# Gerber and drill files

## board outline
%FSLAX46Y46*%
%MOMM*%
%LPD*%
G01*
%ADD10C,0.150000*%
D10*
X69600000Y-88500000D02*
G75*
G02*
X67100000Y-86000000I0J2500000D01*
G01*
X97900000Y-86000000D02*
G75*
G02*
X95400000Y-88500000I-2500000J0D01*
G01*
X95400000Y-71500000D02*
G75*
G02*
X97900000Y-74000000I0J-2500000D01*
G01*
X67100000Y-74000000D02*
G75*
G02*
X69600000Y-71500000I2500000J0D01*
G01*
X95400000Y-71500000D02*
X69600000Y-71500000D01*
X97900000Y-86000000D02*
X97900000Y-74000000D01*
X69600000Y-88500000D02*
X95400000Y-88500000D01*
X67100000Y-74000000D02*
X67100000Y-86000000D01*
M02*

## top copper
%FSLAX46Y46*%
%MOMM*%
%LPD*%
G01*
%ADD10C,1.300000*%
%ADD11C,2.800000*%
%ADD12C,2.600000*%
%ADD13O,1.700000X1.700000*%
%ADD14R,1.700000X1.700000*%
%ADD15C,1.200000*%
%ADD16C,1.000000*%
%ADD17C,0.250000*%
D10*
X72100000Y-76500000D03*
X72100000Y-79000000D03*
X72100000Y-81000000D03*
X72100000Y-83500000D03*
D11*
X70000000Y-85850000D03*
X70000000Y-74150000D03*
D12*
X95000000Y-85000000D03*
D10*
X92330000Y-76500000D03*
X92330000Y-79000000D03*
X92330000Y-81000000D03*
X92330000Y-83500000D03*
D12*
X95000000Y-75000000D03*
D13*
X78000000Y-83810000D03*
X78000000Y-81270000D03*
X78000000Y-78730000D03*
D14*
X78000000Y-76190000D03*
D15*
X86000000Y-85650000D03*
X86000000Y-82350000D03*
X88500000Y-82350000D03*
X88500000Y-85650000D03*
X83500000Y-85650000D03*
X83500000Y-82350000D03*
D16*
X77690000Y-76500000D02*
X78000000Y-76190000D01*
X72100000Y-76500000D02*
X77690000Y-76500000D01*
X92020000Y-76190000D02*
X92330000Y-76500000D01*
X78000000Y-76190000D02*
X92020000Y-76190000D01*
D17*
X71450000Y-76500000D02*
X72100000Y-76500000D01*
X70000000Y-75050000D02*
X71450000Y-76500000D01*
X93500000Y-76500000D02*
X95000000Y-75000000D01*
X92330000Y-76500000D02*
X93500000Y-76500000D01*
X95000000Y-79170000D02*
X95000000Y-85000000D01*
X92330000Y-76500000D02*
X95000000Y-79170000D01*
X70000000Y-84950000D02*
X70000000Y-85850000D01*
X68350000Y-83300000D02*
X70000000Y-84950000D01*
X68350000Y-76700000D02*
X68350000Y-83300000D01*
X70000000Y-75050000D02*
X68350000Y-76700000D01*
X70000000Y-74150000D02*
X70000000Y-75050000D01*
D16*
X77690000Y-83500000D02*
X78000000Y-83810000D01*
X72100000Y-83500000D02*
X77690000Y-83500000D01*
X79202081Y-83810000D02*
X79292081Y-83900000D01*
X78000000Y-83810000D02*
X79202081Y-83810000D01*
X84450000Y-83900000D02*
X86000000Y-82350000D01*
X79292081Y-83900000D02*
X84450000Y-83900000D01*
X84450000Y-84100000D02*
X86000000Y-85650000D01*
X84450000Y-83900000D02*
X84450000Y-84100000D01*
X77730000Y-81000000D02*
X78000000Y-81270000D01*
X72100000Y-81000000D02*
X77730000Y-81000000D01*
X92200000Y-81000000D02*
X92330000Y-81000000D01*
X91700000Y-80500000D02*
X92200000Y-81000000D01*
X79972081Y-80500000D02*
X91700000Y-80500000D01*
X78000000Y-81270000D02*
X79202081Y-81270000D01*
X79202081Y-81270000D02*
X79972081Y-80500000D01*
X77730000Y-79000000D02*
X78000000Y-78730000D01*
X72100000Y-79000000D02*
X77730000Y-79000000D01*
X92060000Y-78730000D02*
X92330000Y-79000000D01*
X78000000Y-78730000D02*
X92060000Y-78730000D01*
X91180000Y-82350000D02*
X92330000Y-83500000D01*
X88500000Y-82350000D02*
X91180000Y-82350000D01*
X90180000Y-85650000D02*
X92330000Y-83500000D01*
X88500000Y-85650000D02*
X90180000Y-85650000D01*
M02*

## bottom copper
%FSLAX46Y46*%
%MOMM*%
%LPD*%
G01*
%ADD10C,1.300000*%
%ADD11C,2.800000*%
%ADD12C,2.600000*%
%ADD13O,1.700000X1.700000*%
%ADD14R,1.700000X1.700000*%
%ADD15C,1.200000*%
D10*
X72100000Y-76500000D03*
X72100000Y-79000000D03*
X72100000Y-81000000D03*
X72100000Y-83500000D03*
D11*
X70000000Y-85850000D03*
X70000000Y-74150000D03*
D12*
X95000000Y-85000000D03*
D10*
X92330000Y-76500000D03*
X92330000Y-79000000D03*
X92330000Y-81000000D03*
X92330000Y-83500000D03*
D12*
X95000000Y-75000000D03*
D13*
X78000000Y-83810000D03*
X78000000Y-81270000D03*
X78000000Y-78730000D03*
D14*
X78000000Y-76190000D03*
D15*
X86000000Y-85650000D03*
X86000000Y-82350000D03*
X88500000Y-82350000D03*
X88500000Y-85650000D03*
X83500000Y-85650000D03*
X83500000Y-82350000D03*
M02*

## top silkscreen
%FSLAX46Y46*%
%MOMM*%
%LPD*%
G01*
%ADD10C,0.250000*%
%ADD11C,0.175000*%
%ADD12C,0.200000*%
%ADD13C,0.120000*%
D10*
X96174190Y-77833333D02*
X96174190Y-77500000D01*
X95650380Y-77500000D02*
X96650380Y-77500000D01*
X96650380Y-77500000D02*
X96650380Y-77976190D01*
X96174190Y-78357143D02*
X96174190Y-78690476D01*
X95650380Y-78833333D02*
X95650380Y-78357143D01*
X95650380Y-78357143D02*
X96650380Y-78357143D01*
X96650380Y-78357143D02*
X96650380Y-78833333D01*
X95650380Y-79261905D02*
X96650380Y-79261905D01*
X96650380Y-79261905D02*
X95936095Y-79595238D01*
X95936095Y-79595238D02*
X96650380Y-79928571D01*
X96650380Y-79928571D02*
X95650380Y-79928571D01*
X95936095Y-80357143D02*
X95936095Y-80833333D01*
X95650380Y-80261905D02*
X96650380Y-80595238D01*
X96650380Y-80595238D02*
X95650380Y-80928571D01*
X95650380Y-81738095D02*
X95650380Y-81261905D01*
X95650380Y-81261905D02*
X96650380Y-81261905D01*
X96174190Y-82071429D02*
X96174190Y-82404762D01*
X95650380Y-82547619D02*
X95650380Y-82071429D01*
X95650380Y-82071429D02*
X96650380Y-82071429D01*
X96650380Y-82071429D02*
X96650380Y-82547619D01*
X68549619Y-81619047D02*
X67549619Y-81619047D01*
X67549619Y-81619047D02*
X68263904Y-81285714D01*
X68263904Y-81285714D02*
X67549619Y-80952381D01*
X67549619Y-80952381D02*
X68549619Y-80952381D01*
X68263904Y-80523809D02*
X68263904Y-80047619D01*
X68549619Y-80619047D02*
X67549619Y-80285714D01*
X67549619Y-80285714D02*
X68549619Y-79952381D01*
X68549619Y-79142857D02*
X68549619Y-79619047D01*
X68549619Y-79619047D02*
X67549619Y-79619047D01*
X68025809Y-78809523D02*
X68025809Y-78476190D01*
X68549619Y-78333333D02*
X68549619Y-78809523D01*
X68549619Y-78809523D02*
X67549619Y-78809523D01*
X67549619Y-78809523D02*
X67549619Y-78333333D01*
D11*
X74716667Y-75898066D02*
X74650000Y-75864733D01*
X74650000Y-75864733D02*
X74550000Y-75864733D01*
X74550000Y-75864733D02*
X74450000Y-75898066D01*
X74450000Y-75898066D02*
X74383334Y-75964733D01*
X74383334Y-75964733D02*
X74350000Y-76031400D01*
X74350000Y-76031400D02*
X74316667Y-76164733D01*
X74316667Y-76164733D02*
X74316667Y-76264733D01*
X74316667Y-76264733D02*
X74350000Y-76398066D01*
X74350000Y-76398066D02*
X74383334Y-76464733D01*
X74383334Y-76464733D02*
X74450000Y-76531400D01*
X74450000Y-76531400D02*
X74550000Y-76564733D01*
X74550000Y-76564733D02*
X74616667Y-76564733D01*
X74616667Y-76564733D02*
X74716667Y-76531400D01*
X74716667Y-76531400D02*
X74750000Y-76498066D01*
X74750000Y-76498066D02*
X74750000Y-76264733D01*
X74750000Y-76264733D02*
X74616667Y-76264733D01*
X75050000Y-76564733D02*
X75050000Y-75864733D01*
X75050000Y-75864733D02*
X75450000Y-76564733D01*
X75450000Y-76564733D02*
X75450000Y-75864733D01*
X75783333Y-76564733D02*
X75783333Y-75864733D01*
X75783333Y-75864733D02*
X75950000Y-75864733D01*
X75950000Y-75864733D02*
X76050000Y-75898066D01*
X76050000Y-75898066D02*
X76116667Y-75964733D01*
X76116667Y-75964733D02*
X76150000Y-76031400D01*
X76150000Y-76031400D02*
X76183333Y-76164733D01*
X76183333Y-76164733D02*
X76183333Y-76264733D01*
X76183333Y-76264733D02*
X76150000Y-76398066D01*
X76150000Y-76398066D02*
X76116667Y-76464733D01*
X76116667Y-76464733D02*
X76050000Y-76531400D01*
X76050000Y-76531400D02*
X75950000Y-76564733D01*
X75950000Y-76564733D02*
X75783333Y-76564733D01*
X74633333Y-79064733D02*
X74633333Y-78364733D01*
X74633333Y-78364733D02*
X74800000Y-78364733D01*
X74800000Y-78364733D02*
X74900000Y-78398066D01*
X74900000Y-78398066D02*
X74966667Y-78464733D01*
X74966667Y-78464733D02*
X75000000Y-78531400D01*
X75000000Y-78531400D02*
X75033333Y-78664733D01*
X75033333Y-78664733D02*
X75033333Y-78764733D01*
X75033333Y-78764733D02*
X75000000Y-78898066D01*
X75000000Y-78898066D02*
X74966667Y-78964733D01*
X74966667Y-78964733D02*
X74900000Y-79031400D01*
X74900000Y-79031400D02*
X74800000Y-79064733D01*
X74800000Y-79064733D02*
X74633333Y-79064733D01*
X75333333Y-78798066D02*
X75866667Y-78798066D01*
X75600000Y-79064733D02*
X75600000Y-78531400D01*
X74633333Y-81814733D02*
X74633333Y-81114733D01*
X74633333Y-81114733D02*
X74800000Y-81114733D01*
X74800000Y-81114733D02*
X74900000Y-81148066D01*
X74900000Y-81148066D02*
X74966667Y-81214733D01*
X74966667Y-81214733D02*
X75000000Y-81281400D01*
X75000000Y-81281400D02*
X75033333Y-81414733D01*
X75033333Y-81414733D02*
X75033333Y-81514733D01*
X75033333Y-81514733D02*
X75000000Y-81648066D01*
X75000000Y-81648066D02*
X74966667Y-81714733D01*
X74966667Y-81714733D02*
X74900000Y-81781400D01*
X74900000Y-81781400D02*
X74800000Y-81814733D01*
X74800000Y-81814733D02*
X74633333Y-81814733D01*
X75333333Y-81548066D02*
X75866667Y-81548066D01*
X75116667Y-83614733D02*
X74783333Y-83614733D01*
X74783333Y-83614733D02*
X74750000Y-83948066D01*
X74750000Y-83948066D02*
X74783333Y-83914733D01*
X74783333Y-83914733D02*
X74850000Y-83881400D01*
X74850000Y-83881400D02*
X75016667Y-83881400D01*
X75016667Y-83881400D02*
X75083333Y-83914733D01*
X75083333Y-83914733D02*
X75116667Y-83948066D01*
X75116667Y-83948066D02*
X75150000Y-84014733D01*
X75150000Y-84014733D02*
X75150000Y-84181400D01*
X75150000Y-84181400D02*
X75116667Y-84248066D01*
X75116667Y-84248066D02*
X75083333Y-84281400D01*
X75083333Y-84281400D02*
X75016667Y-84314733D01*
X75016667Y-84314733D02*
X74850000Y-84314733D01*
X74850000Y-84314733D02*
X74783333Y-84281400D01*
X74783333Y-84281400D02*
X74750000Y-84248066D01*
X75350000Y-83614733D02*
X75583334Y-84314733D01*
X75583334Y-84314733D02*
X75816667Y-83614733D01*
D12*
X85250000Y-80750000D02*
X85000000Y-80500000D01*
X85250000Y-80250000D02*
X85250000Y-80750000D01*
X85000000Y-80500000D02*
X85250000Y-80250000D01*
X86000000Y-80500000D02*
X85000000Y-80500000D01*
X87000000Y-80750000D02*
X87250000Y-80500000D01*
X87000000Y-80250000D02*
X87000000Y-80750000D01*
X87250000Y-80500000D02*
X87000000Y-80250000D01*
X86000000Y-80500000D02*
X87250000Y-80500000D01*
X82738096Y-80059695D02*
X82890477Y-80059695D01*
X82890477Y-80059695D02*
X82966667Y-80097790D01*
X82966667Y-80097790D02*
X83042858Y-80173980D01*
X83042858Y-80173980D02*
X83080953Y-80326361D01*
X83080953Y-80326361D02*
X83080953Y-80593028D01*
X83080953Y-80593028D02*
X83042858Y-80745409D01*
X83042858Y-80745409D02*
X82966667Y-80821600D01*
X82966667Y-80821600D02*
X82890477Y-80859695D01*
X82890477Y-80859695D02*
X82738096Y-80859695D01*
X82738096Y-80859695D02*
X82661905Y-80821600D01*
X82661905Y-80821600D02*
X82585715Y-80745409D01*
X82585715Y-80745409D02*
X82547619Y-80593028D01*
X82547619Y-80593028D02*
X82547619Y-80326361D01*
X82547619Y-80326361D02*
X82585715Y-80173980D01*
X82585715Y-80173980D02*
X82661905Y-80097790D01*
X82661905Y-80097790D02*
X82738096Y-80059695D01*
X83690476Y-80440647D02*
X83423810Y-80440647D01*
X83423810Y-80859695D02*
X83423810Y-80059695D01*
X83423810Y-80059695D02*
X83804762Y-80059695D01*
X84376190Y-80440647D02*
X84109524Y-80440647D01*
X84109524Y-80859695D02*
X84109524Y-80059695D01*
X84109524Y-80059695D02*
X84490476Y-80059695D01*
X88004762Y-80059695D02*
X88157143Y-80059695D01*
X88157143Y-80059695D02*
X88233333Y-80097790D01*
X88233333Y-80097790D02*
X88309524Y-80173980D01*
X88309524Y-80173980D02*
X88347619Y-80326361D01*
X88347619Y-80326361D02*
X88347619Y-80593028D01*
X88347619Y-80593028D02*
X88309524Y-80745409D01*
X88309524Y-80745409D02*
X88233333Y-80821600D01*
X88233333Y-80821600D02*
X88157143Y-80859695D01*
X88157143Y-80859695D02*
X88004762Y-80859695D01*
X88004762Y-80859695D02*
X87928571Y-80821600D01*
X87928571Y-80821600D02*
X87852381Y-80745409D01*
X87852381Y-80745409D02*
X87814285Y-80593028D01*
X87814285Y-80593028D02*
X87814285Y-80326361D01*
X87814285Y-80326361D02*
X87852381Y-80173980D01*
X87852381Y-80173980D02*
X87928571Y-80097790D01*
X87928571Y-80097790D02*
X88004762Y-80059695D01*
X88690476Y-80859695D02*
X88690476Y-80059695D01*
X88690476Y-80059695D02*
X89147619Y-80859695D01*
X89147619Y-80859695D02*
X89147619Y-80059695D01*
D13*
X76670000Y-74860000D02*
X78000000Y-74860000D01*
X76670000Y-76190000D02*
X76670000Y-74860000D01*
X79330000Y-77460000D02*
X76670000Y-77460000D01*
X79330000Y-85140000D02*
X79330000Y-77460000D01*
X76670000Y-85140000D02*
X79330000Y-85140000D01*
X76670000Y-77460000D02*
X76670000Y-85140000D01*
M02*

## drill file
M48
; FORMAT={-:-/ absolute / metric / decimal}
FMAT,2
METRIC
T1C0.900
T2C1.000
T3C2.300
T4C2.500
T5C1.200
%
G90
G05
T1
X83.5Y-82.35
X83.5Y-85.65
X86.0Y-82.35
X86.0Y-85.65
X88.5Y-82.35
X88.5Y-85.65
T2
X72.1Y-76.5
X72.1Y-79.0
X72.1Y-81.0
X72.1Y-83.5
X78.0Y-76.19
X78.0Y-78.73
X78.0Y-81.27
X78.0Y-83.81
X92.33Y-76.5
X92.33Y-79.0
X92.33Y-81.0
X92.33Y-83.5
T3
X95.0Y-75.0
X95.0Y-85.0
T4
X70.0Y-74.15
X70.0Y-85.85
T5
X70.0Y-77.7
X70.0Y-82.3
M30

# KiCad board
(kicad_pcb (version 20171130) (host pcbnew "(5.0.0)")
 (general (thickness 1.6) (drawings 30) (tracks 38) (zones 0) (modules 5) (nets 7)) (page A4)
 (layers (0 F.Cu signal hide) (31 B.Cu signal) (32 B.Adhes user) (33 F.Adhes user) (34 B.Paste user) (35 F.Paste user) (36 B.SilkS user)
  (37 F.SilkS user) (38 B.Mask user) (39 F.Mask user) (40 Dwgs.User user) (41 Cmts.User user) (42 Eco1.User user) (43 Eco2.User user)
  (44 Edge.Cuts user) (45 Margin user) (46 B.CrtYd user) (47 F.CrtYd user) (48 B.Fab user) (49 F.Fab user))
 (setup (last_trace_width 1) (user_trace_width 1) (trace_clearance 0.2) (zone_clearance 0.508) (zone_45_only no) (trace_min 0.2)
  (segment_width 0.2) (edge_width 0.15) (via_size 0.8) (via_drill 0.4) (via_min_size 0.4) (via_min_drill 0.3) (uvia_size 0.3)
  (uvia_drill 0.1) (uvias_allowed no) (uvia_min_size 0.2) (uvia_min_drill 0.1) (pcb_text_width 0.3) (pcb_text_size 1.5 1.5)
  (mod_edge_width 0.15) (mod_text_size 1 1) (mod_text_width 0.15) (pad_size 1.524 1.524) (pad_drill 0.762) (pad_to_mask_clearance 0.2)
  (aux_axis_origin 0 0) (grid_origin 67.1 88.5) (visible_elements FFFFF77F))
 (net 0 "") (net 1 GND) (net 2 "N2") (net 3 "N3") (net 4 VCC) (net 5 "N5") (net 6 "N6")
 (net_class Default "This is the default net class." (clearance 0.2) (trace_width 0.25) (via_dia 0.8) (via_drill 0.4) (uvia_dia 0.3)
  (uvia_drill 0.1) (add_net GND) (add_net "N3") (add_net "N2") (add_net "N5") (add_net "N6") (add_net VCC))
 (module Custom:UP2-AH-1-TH (layer F.Cu) (at 70 80 270)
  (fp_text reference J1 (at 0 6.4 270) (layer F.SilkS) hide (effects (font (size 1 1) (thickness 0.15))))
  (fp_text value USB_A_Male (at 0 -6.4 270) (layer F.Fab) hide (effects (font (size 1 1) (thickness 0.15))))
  (pad 4 thru_hole circle (at -3.5 -2.1 270) (size 1.3 1.3) (drill 1) (layers *.Cu *.Mask) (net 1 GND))
  (pad 3 thru_hole circle (at -1 -2.1 270) (size 1.3 1.3) (drill 1) (layers *.Cu *.Mask) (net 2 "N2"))
  (pad 2 thru_hole circle (at 1 -2.1 270) (size 1.3 1.3) (drill 1) (layers *.Cu *.Mask) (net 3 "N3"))
  (pad 1 thru_hole circle (at 3.5 -2.1 270) (size 1.3 1.3) (drill 1) (layers *.Cu *.Mask) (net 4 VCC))
  (pad 5 thru_hole circle (at 5.85 0 270) (size 2.8 2.8) (drill 2.5) (layers *.Cu *.Mask) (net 1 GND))
  (pad 5 thru_hole circle (at -5.85 0 270) (size 2.8 2.8) (drill 2.5) (layers *.Cu *.Mask) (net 1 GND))
  (pad "" np_thru_hole circle (at 2.3 0 270) (size 1.2 1.2) (drill 1.2) (layers *.Cu *.Mask))
  (pad "" np_thru_hole circle (at -2.3 0 270) (size 1.2 1.2) (drill 1.2) (layers *.Cu *.Mask)))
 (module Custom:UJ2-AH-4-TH (layer F.Cu) (at 95 80 90)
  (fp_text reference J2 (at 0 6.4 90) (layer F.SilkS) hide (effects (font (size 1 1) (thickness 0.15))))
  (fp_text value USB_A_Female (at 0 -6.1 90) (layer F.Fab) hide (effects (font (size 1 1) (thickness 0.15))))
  (pad 5 thru_hole circle (at -5 0 90) (size 2.6 2.6) (drill 2.3) (layers *.Cu *.Mask) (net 1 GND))
  (pad 4 thru_hole circle (at 3.5 -2.67 90) (size 1.3 1.3) (drill 1) (layers *.Cu *.Mask) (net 1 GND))
  (pad 3 thru_hole circle (at 1 -2.67 90) (size 1.3 1.3) (drill 1) (layers *.Cu *.Mask) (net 2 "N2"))
  (pad 2 thru_hole circle (at -1 -2.67 90) (size 1.3 1.3) (drill 1) (layers *.Cu *.Mask) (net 3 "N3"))
  (pad 1 thru_hole circle (at -3.5 -2.67 90) (size 1.3 1.3) (drill 1) (layers *.Cu *.Mask) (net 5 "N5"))
  (pad 5 thru_hole circle (at 5 0 90) (size 2.6 2.6) (drill 2.3) (layers *.Cu *.Mask) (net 1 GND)))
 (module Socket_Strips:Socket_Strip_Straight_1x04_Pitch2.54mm (layer F.Cu) (at 78 76.19)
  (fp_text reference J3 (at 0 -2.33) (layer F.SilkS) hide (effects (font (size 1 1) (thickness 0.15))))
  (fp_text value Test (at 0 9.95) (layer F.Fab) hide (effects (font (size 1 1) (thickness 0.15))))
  (fp_line (start -1.33 -1.33) (end 0 -1.33) (layer F.SilkS) (width 0.12))
  (fp_line (start -1.33 0) (end -1.33 -1.33) (layer F.SilkS) (width 0.12))
  (fp_line (start 1.33 1.27) (end -1.33 1.27) (layer F.SilkS) (width 0.12))
  (fp_line (start 1.33 8.95) (end 1.33 1.27) (layer F.SilkS) (width 0.12))
  (fp_line (start -1.33 8.95) (end 1.33 8.95) (layer F.SilkS) (width 0.12))
  (fp_line (start -1.33 1.27) (end -1.33 8.95) (layer F.SilkS) (width 0.12))
  (pad 4 thru_hole oval (at 0 7.62) (size 1.7 1.7) (drill 1) (layers *.Cu *.Mask) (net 4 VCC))
  (pad 3 thru_hole oval (at 0 5.08) (size 1.7 1.7) (drill 1) (layers *.Cu *.Mask) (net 3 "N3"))
  (pad 2 thru_hole oval (at 0 2.54) (size 1.7 1.7) (drill 1) (layers *.Cu *.Mask) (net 2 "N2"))
  (pad 1 thru_hole rect (at 0 0) (size 1.7 1.7) (drill 1) (layers *.Cu *.Mask) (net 1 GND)))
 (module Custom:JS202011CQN (layer F.Cu) (at 86 84)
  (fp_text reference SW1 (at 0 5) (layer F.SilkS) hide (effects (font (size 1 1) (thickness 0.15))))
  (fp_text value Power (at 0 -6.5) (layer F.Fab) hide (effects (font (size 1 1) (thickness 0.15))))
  (pad 2 thru_hole circle (at 0 1.65) (size 1.2 1.2) (drill 0.9) (layers *.Cu *.Mask) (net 4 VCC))
  (pad 2 thru_hole circle (at 0 -1.65) (size 1.2 1.2) (drill 0.9) (layers *.Cu *.Mask) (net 4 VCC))
  (pad 3 thru_hole circle (at 2.5 -1.65) (size 1.2 1.2) (drill 0.9) (layers *.Cu *.Mask) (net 5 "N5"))
  (pad 3 thru_hole circle (at 2.5 1.65) (size 1.2 1.2) (drill 0.9) (layers *.Cu *.Mask) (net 5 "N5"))
  (pad 1 thru_hole circle (at -2.5 1.65) (size 1.2 1.2) (drill 0.9) (layers *.Cu *.Mask) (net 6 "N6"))
  (pad 1 thru_hole circle (at -2.5 -1.65) (size 1.2 1.2) (drill 0.9) (layers *.Cu *.Mask) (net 6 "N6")))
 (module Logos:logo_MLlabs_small (layer B.Cu) (at 87.25 76.5 180)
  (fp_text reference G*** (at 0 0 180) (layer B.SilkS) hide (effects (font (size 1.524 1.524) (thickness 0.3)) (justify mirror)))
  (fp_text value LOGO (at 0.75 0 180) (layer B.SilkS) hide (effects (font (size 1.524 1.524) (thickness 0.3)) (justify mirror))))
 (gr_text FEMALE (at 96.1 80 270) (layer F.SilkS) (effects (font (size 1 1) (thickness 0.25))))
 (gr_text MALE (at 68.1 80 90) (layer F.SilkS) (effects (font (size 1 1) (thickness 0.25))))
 (gr_arc (start 69.6 86) (end 67.1 86) (angle -90) (layer Edge.Cuts) (width 0.15))
 (gr_arc (start 95.4 86) (end 95.4 88.5) (angle -90) (layer Edge.Cuts) (width 0.15))
 (gr_arc (start 95.4 74) (end 97.9 74) (angle -90) (layer Edge.Cuts) (width 0.15))
 (gr_arc (start 69.6 74) (end 69.6 71.5) (angle -90) (layer Edge.Cuts) (width 0.15))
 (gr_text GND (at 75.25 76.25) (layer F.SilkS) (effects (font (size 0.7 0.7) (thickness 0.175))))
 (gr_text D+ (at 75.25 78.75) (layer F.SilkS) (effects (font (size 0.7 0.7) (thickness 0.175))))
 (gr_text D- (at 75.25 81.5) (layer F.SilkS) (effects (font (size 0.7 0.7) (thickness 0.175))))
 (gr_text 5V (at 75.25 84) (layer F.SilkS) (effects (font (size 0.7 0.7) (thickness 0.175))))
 (gr_line (start 85.25 80.75) (end 85 80.5) (layer F.SilkS) (width 0.2))
 (gr_line (start 85.25 80.25) (end 85.25 80.75) (layer F.SilkS) (width 0.2))
 (gr_line (start 85 80.5) (end 85.25 80.25) (layer F.SilkS) (width 0.2))
 (gr_line (start 86 80.5) (end 85 80.5) (layer F.SilkS) (width 0.2))
 (gr_line (start 87 80.75) (end 87.25 80.5) (layer F.SilkS) (width 0.2))
 (gr_line (start 87 80.25) (end 87 80.75) (layer F.SilkS) (width 0.2))
 (gr_line (start 87.25 80.5) (end 87 80.25) (layer F.SilkS) (width 0.2))
 (gr_line (start 86 80.5) (end 87.25 80.5) (layer F.SilkS) (width 0.2))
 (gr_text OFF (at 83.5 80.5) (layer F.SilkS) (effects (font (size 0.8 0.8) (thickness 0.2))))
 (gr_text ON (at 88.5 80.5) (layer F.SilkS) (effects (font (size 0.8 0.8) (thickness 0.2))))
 (gr_line (start 95.4 71.5) (end 69.6 71.5) (layer Edge.Cuts) (width 0.15))
 (gr_line (start 97.9 86) (end 97.9 74) (layer Edge.Cuts) (width 0.15))
 (gr_line (start 69.6 88.5) (end 95.4 88.5) (layer Edge.Cuts) (width 0.15))
 (gr_line (start 67.1 74) (end 67.1 86) (layer Edge.Cuts) (width 0.15))
 (segment (start 77.69 76.5) (end 78 76.19) (width 1) (layer F.Cu) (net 1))
 (segment (start 72.1 76.5) (end 77.69 76.5) (width 1) (layer F.Cu) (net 1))
 (segment (start 92.02 76.19) (end 92.33 76.5) (width 1) (layer F.Cu) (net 1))
 (segment (start 78 76.19) (end 92.02 76.19) (width 1) (layer F.Cu) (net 1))
 (segment (start 71.45 76.5) (end 72.1 76.5) (width 0.25) (layer F.Cu) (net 1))
 (segment (start 70 75.05) (end 71.45 76.5) (width 0.25) (layer F.Cu) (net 1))
 (segment (start 93.5 76.5) (end 95 75) (width 0.25) (layer F.Cu) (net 1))
 (segment (start 92.33 76.5) (end 93.5 76.5) (width 0.25) (layer F.Cu) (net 1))
 (segment (start 95 79.17) (end 95 85) (width 0.25) (layer F.Cu) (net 1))
 (segment (start 92.33 76.5) (end 95 79.17) (width 0.25) (layer F.Cu) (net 1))
 (segment (start 70 84.95) (end 70 85.85) (width 0.25) (layer F.Cu) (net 1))
 (segment (start 68.35 83.3) (end 70 84.95) (width 0.25) (layer F.Cu) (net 1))
 (segment (start 68.35 76.7) (end 68.35 83.3) (width 0.25) (layer F.Cu) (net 1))
 (segment (start 70 75.05) (end 68.35 76.7) (width 0.25) (layer F.Cu) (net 1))
 (segment (start 70 74.15) (end 70 75.05) (width 0.25) (layer F.Cu) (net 1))
 (segment (start 77.69 83.5) (end 78 83.81) (width 1) (layer F.Cu) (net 4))
 (segment (start 72.1 83.5) (end 77.69 83.5) (width 1) (layer F.Cu) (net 4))
 (segment (start 79.202081 83.81) (end 79.292081 83.9) (width 1) (layer F.Cu) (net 4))
 (segment (start 78 83.81) (end 79.202081 83.81) (width 1) (layer F.Cu) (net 4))
 (segment (start 84.45 83.9) (end 86 82.35) (width 1) (layer F.Cu) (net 4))
 (segment (start 79.292081 83.9) (end 84.45 83.9) (width 1) (layer F.Cu) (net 4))
 (segment (start 84.45 84.1) (end 86 85.65) (width 1) (layer F.Cu) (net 4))
 (segment (start 84.45 83.9) (end 84.45 84.1) (width 1) (layer F.Cu) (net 4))
 (segment (start 77.73 81) (end 78 81.27) (width 1) (layer F.Cu) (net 3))
 (segment (start 72.1 81) (end 77.73 81) (width 1) (layer F.Cu) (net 3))
 (segment (start 92.2 81) (end 92.33 81) (width 1) (layer F.Cu) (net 3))
 (segment (start 91.7 80.5) (end 92.2 81) (width 1) (layer F.Cu) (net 3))
 (segment (start 79.972081 80.5) (end 91.7 80.5) (width 1) (layer F.Cu) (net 3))
 (segment (start 78 81.27) (end 79.202081 81.27) (width 1) (layer F.Cu) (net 3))
 (segment (start 79.202081 81.27) (end 79.972081 80.5) (width 1) (layer F.Cu) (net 3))
 (segment (start 77.73 79) (end 78 78.73) (width 1) (layer F.Cu) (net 2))
 (segment (start 72.1 79) (end 77.73 79) (width 1) (layer F.Cu) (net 2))
 (segment (start 92.06 78.73) (end 92.33 79) (width 1) (layer F.Cu) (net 2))
 (segment (start 78 78.73) (end 92.06 78.73) (width 1) (layer F.Cu) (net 2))
 (segment (start 91.18 82.35) (end 92.33 83.5) (width 1) (layer F.Cu) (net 5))
 (segment (start 88.5 82.35) (end 91.18 82.35) (width 1) (layer F.Cu) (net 5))
 (segment (start 90.18 85.65) (end 92.33 83.5) (width 1) (layer F.Cu) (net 5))
 (segment (start 88.5 85.65) (end 90.18 85.65) (width 1) (layer F.Cu) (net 5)))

